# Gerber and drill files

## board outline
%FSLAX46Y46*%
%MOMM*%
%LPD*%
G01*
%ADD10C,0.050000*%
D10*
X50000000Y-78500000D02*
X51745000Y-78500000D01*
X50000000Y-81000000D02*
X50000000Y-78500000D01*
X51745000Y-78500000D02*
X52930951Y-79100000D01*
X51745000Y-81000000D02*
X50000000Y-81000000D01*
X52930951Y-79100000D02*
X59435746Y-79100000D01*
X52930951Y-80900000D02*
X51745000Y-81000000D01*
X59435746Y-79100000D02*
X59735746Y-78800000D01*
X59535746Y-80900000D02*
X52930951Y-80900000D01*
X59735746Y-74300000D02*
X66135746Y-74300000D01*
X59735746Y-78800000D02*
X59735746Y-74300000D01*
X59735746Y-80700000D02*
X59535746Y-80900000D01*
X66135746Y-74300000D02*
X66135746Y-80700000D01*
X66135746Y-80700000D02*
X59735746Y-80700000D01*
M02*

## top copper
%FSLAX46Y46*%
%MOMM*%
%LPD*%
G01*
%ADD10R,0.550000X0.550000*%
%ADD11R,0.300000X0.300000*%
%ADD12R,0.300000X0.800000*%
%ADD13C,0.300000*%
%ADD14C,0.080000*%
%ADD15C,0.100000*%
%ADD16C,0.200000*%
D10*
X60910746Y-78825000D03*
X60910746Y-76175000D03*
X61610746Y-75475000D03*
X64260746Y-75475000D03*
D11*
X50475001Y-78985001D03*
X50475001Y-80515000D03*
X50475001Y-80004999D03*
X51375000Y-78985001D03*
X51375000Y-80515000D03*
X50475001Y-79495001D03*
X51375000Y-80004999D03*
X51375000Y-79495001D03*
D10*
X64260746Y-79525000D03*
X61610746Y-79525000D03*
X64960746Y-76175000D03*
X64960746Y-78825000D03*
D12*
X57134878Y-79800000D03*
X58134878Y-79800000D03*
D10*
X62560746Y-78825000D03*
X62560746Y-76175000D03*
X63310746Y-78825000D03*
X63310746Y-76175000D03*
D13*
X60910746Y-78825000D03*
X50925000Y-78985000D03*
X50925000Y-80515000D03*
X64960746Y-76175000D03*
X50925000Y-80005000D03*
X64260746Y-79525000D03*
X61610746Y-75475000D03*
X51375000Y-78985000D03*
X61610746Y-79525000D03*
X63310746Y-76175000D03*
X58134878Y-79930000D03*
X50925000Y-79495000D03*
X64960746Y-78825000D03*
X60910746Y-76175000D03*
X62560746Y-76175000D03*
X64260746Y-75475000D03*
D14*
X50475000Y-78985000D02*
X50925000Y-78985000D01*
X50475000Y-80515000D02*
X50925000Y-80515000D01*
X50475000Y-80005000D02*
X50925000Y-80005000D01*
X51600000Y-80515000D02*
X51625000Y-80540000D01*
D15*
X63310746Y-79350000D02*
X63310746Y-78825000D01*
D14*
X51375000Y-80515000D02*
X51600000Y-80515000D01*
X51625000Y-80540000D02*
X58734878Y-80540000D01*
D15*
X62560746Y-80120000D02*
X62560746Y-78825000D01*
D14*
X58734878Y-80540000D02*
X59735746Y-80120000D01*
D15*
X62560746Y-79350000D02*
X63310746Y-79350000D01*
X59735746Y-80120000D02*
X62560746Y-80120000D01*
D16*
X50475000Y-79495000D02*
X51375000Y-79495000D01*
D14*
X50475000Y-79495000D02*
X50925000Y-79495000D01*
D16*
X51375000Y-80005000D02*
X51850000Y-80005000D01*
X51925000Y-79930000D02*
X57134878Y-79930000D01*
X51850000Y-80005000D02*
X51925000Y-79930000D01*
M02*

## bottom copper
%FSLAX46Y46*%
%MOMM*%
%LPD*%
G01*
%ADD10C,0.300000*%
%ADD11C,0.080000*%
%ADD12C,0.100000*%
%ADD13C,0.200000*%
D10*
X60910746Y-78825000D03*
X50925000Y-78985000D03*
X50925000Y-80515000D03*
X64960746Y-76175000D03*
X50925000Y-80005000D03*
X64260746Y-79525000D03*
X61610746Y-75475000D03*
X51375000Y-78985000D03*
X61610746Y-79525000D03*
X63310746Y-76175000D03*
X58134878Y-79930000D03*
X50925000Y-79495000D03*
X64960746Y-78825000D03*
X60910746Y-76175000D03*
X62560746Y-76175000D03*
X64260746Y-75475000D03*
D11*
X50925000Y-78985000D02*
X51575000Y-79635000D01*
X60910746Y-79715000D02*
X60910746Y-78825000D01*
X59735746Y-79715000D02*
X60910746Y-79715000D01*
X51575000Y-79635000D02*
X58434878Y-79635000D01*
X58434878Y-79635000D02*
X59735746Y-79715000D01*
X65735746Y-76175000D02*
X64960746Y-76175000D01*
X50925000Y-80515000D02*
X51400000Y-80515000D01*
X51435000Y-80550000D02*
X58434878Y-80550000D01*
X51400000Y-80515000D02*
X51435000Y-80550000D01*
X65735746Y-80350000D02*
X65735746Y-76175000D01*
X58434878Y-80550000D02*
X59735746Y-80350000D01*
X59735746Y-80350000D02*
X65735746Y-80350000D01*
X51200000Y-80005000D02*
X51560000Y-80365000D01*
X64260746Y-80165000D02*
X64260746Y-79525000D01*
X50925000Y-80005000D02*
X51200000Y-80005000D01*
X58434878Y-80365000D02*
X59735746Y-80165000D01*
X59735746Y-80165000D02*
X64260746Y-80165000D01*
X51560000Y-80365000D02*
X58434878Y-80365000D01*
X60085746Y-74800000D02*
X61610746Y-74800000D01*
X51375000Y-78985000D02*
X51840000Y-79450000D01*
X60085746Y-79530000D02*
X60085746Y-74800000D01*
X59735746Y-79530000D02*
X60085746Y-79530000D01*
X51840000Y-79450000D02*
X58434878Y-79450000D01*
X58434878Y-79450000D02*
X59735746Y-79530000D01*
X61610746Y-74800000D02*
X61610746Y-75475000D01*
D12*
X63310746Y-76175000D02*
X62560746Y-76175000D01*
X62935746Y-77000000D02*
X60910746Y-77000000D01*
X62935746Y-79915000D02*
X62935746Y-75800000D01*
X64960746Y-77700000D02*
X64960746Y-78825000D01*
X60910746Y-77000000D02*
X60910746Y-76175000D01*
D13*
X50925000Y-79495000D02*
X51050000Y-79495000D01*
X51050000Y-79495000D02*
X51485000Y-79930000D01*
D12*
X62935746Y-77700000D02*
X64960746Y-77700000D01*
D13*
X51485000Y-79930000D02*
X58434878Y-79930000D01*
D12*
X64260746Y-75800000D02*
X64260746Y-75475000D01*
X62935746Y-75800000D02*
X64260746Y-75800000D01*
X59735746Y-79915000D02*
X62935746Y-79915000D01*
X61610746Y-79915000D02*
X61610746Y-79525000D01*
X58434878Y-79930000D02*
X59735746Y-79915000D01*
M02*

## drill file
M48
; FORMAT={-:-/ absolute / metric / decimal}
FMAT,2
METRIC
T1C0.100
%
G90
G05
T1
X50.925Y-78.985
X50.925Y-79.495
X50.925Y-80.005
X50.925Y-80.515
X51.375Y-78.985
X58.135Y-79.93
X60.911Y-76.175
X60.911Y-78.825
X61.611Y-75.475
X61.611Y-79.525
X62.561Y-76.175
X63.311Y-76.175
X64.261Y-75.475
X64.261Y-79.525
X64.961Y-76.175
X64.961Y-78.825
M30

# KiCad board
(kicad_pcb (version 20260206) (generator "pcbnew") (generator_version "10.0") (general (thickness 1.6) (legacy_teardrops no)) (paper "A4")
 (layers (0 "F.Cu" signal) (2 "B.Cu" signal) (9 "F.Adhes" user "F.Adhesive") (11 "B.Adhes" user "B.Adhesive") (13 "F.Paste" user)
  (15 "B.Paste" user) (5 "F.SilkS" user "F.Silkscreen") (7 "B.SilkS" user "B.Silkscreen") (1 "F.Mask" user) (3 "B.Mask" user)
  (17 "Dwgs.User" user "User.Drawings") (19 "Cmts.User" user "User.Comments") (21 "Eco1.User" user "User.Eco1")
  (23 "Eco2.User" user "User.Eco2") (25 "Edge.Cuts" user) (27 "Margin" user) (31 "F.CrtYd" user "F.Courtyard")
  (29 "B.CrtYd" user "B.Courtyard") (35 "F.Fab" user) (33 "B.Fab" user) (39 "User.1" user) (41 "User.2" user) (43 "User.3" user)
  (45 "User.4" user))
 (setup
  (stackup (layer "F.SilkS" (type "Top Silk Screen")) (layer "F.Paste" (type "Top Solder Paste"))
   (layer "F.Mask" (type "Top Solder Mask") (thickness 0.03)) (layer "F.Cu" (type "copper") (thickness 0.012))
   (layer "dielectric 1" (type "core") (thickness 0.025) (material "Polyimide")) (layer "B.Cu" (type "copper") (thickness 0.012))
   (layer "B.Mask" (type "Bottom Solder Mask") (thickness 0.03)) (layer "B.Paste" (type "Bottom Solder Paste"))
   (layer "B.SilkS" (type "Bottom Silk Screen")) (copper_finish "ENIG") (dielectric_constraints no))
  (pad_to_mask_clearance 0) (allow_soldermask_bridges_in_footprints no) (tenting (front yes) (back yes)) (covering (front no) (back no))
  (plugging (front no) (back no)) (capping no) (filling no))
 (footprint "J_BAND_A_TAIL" (layer "F.Cu") (at 50.9 79.75)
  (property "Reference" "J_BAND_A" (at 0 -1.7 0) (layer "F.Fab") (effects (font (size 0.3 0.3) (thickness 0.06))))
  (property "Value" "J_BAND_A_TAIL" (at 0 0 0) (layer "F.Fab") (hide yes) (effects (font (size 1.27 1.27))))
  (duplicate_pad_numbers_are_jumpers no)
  (pad "1" smd rect (at -0.424999 -0.764999) (size 0.3 0.3) (layers "F.Cu" "F.Mask") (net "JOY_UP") (solder_mask_margin 0.05)
   (thermal_bridge_angle 45))
  (pad "2" smd rect (at -0.424999 0.765) (size 0.3 0.3) (layers "F.Cu" "F.Mask") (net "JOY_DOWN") (solder_mask_margin 0.05)
   (thermal_bridge_angle 45))
  (pad "3" smd rect (at -0.424999 0.254999) (size 0.3 0.3) (layers "F.Cu" "F.Mask") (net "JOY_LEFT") (solder_mask_margin 0.05)
   (thermal_bridge_angle 45))
  (pad "4" smd rect (at 0.475 -0.764999) (size 0.3 0.3) (layers "F.Cu" "F.Mask") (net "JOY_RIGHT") (solder_mask_margin 0.05)
   (thermal_bridge_angle 45))
  (pad "5" smd rect (at 0.475 0.765) (size 0.3 0.3) (layers "F.Cu" "F.Mask") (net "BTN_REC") (solder_mask_margin 0.05)
   (thermal_bridge_angle 45))
  (pad "6" smd rect (at -0.424999 -0.254999) (size 0.3 0.3) (layers "F.Cu" "F.Mask") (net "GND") (solder_mask_margin 0.05)
   (thermal_bridge_angle 45))
  (pad "7" smd rect (at 0.475 0.254999) (size 0.3 0.3) (layers "F.Cu" "F.Mask") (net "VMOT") (solder_mask_margin 0.05)
   (thermal_bridge_angle 45))
  (pad "8" smd rect (at 0.475 -0.254999) (size 0.3 0.3) (layers "F.Cu" "F.Mask") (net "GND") (solder_mask_margin 0.05)
   (thermal_bridge_angle 45)))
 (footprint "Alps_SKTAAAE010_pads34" (layer "F.Cu") (at 62.935746 75.1)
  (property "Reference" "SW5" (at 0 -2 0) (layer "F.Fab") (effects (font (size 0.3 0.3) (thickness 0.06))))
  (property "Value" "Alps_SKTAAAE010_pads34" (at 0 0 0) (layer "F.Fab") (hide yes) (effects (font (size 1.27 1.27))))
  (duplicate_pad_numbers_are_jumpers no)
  (pad "3" smd rect (at -1.325 0.375) (size 0.55 0.55) (layers "F.Cu" "F.Mask") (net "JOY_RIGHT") (solder_mask_margin 0.05)
   (thermal_bridge_angle 45))
  (pad "4" smd rect (at 1.325 0.375) (size 0.55 0.55) (layers "F.Cu" "F.Mask") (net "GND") (solder_mask_margin 0.05)
   (thermal_bridge_angle 45)))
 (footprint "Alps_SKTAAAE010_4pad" (layer "F.Cu") (at 62.935746 77.5 90)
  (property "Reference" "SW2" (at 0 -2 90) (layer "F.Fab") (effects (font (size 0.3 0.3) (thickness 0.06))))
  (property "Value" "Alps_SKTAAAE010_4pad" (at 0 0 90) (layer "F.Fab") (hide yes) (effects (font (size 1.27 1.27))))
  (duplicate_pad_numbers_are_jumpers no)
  (pad "1" smd rect (at -1.325 -0.375 90) (size 0.55 0.55) (layers "F.Cu" "F.Mask") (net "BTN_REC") (solder_mask_margin 0.05)
   (thermal_bridge_angle 45))
  (pad "2" smd rect (at 1.325 -0.375 90) (size 0.55 0.55) (layers "F.Cu" "F.Mask") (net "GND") (solder_mask_margin 0.05)
   (thermal_bridge_angle 45))
  (pad "3" smd rect (at -1.325 0.375 90) (size 0.55 0.55) (layers "F.Cu" "F.Mask") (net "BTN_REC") (solder_mask_margin 0.05)
   (thermal_bridge_angle 45))
  (pad "4" smd rect (at 1.325 0.375 90) (size 0.55 0.55) (layers "F.Cu" "F.Mask") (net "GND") (solder_mask_margin 0.05)
   (thermal_bridge_angle 45)))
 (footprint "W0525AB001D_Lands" (layer "F.Cu") (at 57.634878 79.93)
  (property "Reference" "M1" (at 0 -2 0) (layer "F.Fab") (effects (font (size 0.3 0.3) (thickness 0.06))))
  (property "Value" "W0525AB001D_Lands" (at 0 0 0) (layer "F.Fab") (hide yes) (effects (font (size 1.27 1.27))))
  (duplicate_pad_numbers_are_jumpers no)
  (pad "1" smd rect (at -0.5 -0.13) (size 0.3 0.8) (layers "F.Cu" "F.Mask") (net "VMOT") (solder_mask_margin 0.05) (thermal_bridge_angle 45))
  (pad "2" smd rect (at 0.5 -0.13) (size 0.3 0.8) (layers "F.Cu" "F.Mask") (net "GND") (solder_mask_margin 0.05) (thermal_bridge_angle 45)))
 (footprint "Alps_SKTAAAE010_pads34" (layer "F.Cu") (at 60.535746 77.5 90)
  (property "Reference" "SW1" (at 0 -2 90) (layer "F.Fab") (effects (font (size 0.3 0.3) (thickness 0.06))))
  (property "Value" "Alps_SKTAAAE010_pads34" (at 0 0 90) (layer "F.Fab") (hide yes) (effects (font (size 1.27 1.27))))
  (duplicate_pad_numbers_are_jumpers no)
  (pad "3" smd rect (at -1.325 0.375 90) (size 0.55 0.55) (layers "F.Cu" "F.Mask") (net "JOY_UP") (solder_mask_margin 0.05)
   (thermal_bridge_angle 45))
  (pad "4" smd rect (at 1.325 0.375 90) (size 0.55 0.55) (layers "F.Cu" "F.Mask") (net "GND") (solder_mask_margin 0.05)
   (thermal_bridge_angle 45)))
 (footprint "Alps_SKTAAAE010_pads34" (layer "F.Cu") (at 62.935746 79.9 180)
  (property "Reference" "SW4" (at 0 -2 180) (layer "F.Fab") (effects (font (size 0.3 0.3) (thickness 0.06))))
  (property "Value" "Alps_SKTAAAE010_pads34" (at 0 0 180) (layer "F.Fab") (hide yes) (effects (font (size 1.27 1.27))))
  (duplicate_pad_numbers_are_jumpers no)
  (pad "3" smd rect (at -1.325 0.375 180) (size 0.55 0.55) (layers "F.Cu" "F.Mask") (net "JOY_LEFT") (solder_mask_margin 0.05)
   (thermal_bridge_angle 45))
  (pad "4" smd rect (at 1.325 0.375 180) (size 0.55 0.55) (layers "F.Cu" "F.Mask") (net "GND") (solder_mask_margin 0.05)
   (thermal_bridge_angle 45)))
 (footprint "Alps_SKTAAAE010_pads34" (layer "F.Cu") (at 65.335746 77.5 -90)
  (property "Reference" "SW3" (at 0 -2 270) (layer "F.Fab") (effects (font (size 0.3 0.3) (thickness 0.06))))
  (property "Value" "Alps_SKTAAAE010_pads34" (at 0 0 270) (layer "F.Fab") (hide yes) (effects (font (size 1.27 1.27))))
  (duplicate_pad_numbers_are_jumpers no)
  (pad "3" smd rect (at -1.325 0.375 270) (size 0.55 0.55) (layers "F.Cu" "F.Mask") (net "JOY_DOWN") (solder_mask_margin 0.05)
   (thermal_bridge_angle 45))
  (pad "4" smd rect (at 1.325 0.375 270) (size 0.55 0.55) (layers "F.Cu" "F.Mask") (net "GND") (solder_mask_margin 0.05)
   (thermal_bridge_angle 45)))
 (gr_line (start 50 78.5) (end 51.745 78.5) (stroke (width 0.05) (type default)) (layer "Edge.Cuts"))
 (gr_line (start 50 81) (end 50 78.5) (stroke (width 0.05) (type default)) (layer "Edge.Cuts"))
 (gr_line (start 51.745 78.5) (end 52.930951 79.1) (stroke (width 0.05) (type default)) (layer "Edge.Cuts"))
 (gr_line (start 51.745 81) (end 50 81) (stroke (width 0.05) (type default)) (layer "Edge.Cuts"))
 (gr_line (start 52.930951 79.1) (end 59.435746 79.1) (stroke (width 0.05) (type default)) (layer "Edge.Cuts"))
 (gr_line (start 52.930951 80.9) (end 51.745 81) (stroke (width 0.05) (type default)) (layer "Edge.Cuts"))
 (gr_line (start 59.435746 79.1) (end 59.735746 78.8) (stroke (width 0.05) (type default)) (layer "Edge.Cuts"))
 (gr_line (start 59.535746 80.9) (end 52.930951 80.9) (stroke (width 0.05) (type default)) (layer "Edge.Cuts"))
 (gr_line (start 59.735746 74.3) (end 66.135746 74.3) (stroke (width 0.05) (type default)) (layer "Edge.Cuts"))
 (gr_line (start 59.735746 78.8) (end 59.735746 74.3) (stroke (width 0.05) (type default)) (layer "Edge.Cuts"))
 (gr_line (start 59.735746 80.7) (end 59.535746 80.9) (stroke (width 0.05) (type default)) (layer "Edge.Cuts"))
 (gr_line (start 66.135746 74.3) (end 66.135746 80.7) (stroke (width 0.05) (type default)) (layer "Edge.Cuts"))
 (gr_line (start 66.135746 80.7) (end 59.735746 80.7) (stroke (width 0.05) (type default)) (layer "Edge.Cuts"))
 (segment (start 50.475 78.985) (end 50.925 78.985) (width 0.08) (layer "F.Cu") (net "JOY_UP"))
 (via (at 60.910746 78.825) (size 0.3) (drill 0.1) (layers "F.Cu" "B.Cu") (tenting (front yes) (back yes)) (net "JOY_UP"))
 (via (at 50.925 78.985) (size 0.3) (drill 0.1) (layers "F.Cu" "B.Cu") (tenting (front yes) (back yes)) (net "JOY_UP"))
 (segment (start 60.910746 79.715) (end 60.910746 78.825) (width 0.08) (layer "B.Cu") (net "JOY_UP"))
 (segment (start 58.434878 79.635) (end 59.735746 79.715) (width 0.08) (layer "B.Cu") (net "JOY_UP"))
 (segment (start 59.735746 79.715) (end 60.910746 79.715) (width 0.08) (layer "B.Cu") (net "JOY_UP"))
 (segment (start 50.925 78.985) (end 51.575 79.635) (width 0.08) (layer "B.Cu") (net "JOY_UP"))
 (segment (start 51.575 79.635) (end 58.434878 79.635) (width 0.08) (layer "B.Cu") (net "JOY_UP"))
 (segment (start 50.475 80.515) (end 50.925 80.515) (width 0.08) (layer "F.Cu") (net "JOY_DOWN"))
 (via (at 50.925 80.515) (size 0.3) (drill 0.1) (layers "F.Cu" "B.Cu") (tenting (front yes) (back yes)) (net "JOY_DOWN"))
 (via (at 64.960746 76.175) (size 0.3) (drill 0.1) (layers "F.Cu" "B.Cu") (tenting (front yes) (back yes)) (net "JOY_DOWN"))
 (segment (start 51.435 80.55) (end 58.434878 80.55) (width 0.08) (layer "B.Cu") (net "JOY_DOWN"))
 (segment (start 50.925 80.515) (end 51.4 80.515) (width 0.08) (layer "B.Cu") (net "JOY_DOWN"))
 (segment (start 65.735746 80.35) (end 65.735746 76.175) (width 0.08) (layer "B.Cu") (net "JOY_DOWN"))
 (segment (start 58.434878 80.55) (end 59.735746 80.35) (width 0.08) (layer "B.Cu") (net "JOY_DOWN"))
 (segment (start 51.4 80.515) (end 51.435 80.55) (width 0.08) (layer "B.Cu") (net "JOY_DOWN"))
 (segment (start 65.735746 76.175) (end 64.960746 76.175) (width 0.08) (layer "B.Cu") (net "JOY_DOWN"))
 (segment (start 59.735746 80.35) (end 65.735746 80.35) (width 0.08) (layer "B.Cu") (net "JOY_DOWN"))
 (segment (start 50.475 80.005) (end 50.925 80.005) (width 0.08) (layer "F.Cu") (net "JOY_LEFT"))
 (via (at 50.925 80.005) (size 0.3) (drill 0.1) (layers "F.Cu" "B.Cu") (tenting (front yes) (back yes)) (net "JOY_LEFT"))
 (via (at 64.260746 79.525) (size 0.3) (drill 0.1) (layers "F.Cu" "B.Cu") (tenting (front yes) (back yes)) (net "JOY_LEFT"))
 (segment (start 51.2 80.005) (end 51.56 80.365) (width 0.08) (layer "B.Cu") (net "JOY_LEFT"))
 (segment (start 51.56 80.365) (end 58.434878 80.365) (width 0.08) (layer "B.Cu") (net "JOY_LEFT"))
 (segment (start 64.260746 80.165) (end 64.260746 79.525) (width 0.08) (layer "B.Cu") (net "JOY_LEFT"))
 (segment (start 59.735746 80.165) (end 64.260746 80.165) (width 0.08) (layer "B.Cu") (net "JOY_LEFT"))
 (segment (start 50.925 80.005) (end 51.2 80.005) (width 0.08) (layer "B.Cu") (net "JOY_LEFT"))
 (segment (start 58.434878 80.365) (end 59.735746 80.165) (width 0.08) (layer "B.Cu") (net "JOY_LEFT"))
 (via (at 51.375 78.985) (size 0.3) (drill 0.1) (layers "F.Cu" "B.Cu") (tenting (front yes) (back yes)) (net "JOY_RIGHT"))
 (via (at 61.610746 75.475) (size 0.3) (drill 0.1) (layers "F.Cu" "B.Cu") (tenting (front yes) (back yes)) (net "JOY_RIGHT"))
 (segment (start 51.375 78.985) (end 51.84 79.45) (width 0.08) (layer "B.Cu") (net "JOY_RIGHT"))
 (segment (start 61.610746 74.8) (end 61.610746 75.475) (width 0.08) (layer "B.Cu") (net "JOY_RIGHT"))
 (segment (start 60.085746 79.53) (end 60.085746 74.8) (width 0.08) (layer "B.Cu") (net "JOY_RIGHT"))
 (segment (start 58.434878 79.45) (end 59.735746 79.53) (width 0.08) (layer "B.Cu") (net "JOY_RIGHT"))
 (segment (start 59.735746 79.53) (end 60.085746 79.53) (width 0.08) (layer "B.Cu") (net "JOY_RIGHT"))
 (segment (start 60.085746 74.8) (end 61.610746 74.8) (width 0.08) (layer "B.Cu") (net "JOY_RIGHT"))
 (segment (start 51.84 79.45) (end 58.434878 79.45) (width 0.08) (layer "B.Cu") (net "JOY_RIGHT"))
 (segment (start 51.625 80.54) (end 58.734878 80.54) (width 0.08) (layer "F.Cu") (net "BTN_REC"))
 (segment (start 63.310746 79.35) (end 63.310746 78.825) (width 0.1) (layer "F.Cu") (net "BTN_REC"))
 (segment (start 58.734878 80.54) (end 59.735746 80.12) (width 0.08) (layer "F.Cu") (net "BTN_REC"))
 (segment (start 51.375 80.515) (end 51.6 80.515) (width 0.08) (layer "F.Cu") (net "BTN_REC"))
 (segment (start 62.560746 79.35) (end 63.310746 79.35) (width 0.1) (layer "F.Cu") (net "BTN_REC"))
 (segment (start 51.6 80.515) (end 51.625 80.54) (width 0.08) (layer "F.Cu") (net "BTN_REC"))
 (segment (start 59.735746 80.12) (end 62.560746 80.12) (width 0.1) (layer "F.Cu") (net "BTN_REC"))
 (segment (start 62.560746 80.12) (end 62.560746 78.825) (width 0.1) (layer "F.Cu") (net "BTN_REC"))
 (segment (start 50.475 79.495) (end 50.925 79.495) (width 0.08) (layer "F.Cu") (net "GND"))
 (segment (start 50.475 79.495) (end 51.375 79.495) (width 0.2) (layer "F.Cu") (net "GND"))
 (via (at 64.260746 75.475) (size 0.3) (drill 0.1) (layers "F.Cu" "B.Cu") (tenting (front yes) (back yes)) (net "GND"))
 (via (at 63.310746 76.175) (size 0.3) (drill 0.1) (layers "F.Cu" "B.Cu") (tenting (front yes) (back yes)) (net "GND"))
 (via (at 50.925 79.495) (size 0.3) (drill 0.1) (layers "F.Cu" "B.Cu") (tenting (front yes) (back yes)) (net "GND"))
 (via (at 61.610746 79.525) (size 0.3) (drill 0.1) (layers "F.Cu" "B.Cu") (tenting (front yes) (back yes)) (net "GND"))
 (via (at 62.560746 76.175) (size 0.3) (drill 0.1) (layers "F.Cu" "B.Cu") (tenting (front yes) (back yes)) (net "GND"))
 (via (at 64.960746 78.825) (size 0.3) (drill 0.1) (layers "F.Cu" "B.Cu") (tenting (front yes) (back yes)) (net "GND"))
 (via (at 60.910746 76.175) (size 0.3) (drill 0.1) (layers "F.Cu" "B.Cu") (tenting (front yes) (back yes)) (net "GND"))
 (via (at 58.134878 79.93) (size 0.3) (drill 0.1) (layers "F.Cu" "B.Cu") (tenting (front yes) (back yes)) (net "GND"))
 (segment (start 51.485 79.93) (end 58.434878 79.93) (width 0.2) (layer "B.Cu") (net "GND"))
 (segment (start 62.935746 77.7) (end 64.960746 77.7) (width 0.1) (layer "B.Cu") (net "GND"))
 (segment (start 62.935746 77) (end 60.910746 77) (width 0.1) (layer "B.Cu") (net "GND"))
 (segment (start 59.735746 79.915) (end 62.935746 79.915) (width 0.1) (layer "B.Cu") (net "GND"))
 (segment (start 62.935746 75.8) (end 64.260746 75.8) (width 0.1) (layer "B.Cu") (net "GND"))
 (segment (start 58.434878 79.93) (end 59.735746 79.915) (width 0.1) (layer "B.Cu") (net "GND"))
 (segment (start 64.960746 77.7) (end 64.960746 78.825) (width 0.1) (layer "B.Cu") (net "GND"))
 (segment (start 61.610746 79.915) (end 61.610746 79.525) (width 0.1) (layer "B.Cu") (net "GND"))
 (segment (start 62.935746 79.915) (end 62.935746 75.8) (width 0.1) (layer "B.Cu") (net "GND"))
 (segment (start 64.260746 75.8) (end 64.260746 75.475) (width 0.1) (layer "B.Cu") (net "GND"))
 (segment (start 50.925 79.495) (end 51.05 79.495) (width 0.2) (layer "B.Cu") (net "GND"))
 (segment (start 63.310746 76.175) (end 62.560746 76.175) (width 0.1) (layer "B.Cu") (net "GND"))
 (segment (start 51.05 79.495) (end 51.485 79.93) (width 0.2) (layer "B.Cu") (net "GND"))
 (segment (start 60.910746 77) (end 60.910746 76.175) (width 0.1) (layer "B.Cu") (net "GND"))
 (segment (start 51.925 79.93) (end 57.134878 79.93) (width 0.2) (layer "F.Cu") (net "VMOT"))
 (segment (start 51.375 80.005) (end 51.85 80.005) (width 0.2) (layer "F.Cu") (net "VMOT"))
 (segment (start 51.85 80.005) (end 51.925 79.93) (width 0.2) (layer "F.Cu") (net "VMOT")))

